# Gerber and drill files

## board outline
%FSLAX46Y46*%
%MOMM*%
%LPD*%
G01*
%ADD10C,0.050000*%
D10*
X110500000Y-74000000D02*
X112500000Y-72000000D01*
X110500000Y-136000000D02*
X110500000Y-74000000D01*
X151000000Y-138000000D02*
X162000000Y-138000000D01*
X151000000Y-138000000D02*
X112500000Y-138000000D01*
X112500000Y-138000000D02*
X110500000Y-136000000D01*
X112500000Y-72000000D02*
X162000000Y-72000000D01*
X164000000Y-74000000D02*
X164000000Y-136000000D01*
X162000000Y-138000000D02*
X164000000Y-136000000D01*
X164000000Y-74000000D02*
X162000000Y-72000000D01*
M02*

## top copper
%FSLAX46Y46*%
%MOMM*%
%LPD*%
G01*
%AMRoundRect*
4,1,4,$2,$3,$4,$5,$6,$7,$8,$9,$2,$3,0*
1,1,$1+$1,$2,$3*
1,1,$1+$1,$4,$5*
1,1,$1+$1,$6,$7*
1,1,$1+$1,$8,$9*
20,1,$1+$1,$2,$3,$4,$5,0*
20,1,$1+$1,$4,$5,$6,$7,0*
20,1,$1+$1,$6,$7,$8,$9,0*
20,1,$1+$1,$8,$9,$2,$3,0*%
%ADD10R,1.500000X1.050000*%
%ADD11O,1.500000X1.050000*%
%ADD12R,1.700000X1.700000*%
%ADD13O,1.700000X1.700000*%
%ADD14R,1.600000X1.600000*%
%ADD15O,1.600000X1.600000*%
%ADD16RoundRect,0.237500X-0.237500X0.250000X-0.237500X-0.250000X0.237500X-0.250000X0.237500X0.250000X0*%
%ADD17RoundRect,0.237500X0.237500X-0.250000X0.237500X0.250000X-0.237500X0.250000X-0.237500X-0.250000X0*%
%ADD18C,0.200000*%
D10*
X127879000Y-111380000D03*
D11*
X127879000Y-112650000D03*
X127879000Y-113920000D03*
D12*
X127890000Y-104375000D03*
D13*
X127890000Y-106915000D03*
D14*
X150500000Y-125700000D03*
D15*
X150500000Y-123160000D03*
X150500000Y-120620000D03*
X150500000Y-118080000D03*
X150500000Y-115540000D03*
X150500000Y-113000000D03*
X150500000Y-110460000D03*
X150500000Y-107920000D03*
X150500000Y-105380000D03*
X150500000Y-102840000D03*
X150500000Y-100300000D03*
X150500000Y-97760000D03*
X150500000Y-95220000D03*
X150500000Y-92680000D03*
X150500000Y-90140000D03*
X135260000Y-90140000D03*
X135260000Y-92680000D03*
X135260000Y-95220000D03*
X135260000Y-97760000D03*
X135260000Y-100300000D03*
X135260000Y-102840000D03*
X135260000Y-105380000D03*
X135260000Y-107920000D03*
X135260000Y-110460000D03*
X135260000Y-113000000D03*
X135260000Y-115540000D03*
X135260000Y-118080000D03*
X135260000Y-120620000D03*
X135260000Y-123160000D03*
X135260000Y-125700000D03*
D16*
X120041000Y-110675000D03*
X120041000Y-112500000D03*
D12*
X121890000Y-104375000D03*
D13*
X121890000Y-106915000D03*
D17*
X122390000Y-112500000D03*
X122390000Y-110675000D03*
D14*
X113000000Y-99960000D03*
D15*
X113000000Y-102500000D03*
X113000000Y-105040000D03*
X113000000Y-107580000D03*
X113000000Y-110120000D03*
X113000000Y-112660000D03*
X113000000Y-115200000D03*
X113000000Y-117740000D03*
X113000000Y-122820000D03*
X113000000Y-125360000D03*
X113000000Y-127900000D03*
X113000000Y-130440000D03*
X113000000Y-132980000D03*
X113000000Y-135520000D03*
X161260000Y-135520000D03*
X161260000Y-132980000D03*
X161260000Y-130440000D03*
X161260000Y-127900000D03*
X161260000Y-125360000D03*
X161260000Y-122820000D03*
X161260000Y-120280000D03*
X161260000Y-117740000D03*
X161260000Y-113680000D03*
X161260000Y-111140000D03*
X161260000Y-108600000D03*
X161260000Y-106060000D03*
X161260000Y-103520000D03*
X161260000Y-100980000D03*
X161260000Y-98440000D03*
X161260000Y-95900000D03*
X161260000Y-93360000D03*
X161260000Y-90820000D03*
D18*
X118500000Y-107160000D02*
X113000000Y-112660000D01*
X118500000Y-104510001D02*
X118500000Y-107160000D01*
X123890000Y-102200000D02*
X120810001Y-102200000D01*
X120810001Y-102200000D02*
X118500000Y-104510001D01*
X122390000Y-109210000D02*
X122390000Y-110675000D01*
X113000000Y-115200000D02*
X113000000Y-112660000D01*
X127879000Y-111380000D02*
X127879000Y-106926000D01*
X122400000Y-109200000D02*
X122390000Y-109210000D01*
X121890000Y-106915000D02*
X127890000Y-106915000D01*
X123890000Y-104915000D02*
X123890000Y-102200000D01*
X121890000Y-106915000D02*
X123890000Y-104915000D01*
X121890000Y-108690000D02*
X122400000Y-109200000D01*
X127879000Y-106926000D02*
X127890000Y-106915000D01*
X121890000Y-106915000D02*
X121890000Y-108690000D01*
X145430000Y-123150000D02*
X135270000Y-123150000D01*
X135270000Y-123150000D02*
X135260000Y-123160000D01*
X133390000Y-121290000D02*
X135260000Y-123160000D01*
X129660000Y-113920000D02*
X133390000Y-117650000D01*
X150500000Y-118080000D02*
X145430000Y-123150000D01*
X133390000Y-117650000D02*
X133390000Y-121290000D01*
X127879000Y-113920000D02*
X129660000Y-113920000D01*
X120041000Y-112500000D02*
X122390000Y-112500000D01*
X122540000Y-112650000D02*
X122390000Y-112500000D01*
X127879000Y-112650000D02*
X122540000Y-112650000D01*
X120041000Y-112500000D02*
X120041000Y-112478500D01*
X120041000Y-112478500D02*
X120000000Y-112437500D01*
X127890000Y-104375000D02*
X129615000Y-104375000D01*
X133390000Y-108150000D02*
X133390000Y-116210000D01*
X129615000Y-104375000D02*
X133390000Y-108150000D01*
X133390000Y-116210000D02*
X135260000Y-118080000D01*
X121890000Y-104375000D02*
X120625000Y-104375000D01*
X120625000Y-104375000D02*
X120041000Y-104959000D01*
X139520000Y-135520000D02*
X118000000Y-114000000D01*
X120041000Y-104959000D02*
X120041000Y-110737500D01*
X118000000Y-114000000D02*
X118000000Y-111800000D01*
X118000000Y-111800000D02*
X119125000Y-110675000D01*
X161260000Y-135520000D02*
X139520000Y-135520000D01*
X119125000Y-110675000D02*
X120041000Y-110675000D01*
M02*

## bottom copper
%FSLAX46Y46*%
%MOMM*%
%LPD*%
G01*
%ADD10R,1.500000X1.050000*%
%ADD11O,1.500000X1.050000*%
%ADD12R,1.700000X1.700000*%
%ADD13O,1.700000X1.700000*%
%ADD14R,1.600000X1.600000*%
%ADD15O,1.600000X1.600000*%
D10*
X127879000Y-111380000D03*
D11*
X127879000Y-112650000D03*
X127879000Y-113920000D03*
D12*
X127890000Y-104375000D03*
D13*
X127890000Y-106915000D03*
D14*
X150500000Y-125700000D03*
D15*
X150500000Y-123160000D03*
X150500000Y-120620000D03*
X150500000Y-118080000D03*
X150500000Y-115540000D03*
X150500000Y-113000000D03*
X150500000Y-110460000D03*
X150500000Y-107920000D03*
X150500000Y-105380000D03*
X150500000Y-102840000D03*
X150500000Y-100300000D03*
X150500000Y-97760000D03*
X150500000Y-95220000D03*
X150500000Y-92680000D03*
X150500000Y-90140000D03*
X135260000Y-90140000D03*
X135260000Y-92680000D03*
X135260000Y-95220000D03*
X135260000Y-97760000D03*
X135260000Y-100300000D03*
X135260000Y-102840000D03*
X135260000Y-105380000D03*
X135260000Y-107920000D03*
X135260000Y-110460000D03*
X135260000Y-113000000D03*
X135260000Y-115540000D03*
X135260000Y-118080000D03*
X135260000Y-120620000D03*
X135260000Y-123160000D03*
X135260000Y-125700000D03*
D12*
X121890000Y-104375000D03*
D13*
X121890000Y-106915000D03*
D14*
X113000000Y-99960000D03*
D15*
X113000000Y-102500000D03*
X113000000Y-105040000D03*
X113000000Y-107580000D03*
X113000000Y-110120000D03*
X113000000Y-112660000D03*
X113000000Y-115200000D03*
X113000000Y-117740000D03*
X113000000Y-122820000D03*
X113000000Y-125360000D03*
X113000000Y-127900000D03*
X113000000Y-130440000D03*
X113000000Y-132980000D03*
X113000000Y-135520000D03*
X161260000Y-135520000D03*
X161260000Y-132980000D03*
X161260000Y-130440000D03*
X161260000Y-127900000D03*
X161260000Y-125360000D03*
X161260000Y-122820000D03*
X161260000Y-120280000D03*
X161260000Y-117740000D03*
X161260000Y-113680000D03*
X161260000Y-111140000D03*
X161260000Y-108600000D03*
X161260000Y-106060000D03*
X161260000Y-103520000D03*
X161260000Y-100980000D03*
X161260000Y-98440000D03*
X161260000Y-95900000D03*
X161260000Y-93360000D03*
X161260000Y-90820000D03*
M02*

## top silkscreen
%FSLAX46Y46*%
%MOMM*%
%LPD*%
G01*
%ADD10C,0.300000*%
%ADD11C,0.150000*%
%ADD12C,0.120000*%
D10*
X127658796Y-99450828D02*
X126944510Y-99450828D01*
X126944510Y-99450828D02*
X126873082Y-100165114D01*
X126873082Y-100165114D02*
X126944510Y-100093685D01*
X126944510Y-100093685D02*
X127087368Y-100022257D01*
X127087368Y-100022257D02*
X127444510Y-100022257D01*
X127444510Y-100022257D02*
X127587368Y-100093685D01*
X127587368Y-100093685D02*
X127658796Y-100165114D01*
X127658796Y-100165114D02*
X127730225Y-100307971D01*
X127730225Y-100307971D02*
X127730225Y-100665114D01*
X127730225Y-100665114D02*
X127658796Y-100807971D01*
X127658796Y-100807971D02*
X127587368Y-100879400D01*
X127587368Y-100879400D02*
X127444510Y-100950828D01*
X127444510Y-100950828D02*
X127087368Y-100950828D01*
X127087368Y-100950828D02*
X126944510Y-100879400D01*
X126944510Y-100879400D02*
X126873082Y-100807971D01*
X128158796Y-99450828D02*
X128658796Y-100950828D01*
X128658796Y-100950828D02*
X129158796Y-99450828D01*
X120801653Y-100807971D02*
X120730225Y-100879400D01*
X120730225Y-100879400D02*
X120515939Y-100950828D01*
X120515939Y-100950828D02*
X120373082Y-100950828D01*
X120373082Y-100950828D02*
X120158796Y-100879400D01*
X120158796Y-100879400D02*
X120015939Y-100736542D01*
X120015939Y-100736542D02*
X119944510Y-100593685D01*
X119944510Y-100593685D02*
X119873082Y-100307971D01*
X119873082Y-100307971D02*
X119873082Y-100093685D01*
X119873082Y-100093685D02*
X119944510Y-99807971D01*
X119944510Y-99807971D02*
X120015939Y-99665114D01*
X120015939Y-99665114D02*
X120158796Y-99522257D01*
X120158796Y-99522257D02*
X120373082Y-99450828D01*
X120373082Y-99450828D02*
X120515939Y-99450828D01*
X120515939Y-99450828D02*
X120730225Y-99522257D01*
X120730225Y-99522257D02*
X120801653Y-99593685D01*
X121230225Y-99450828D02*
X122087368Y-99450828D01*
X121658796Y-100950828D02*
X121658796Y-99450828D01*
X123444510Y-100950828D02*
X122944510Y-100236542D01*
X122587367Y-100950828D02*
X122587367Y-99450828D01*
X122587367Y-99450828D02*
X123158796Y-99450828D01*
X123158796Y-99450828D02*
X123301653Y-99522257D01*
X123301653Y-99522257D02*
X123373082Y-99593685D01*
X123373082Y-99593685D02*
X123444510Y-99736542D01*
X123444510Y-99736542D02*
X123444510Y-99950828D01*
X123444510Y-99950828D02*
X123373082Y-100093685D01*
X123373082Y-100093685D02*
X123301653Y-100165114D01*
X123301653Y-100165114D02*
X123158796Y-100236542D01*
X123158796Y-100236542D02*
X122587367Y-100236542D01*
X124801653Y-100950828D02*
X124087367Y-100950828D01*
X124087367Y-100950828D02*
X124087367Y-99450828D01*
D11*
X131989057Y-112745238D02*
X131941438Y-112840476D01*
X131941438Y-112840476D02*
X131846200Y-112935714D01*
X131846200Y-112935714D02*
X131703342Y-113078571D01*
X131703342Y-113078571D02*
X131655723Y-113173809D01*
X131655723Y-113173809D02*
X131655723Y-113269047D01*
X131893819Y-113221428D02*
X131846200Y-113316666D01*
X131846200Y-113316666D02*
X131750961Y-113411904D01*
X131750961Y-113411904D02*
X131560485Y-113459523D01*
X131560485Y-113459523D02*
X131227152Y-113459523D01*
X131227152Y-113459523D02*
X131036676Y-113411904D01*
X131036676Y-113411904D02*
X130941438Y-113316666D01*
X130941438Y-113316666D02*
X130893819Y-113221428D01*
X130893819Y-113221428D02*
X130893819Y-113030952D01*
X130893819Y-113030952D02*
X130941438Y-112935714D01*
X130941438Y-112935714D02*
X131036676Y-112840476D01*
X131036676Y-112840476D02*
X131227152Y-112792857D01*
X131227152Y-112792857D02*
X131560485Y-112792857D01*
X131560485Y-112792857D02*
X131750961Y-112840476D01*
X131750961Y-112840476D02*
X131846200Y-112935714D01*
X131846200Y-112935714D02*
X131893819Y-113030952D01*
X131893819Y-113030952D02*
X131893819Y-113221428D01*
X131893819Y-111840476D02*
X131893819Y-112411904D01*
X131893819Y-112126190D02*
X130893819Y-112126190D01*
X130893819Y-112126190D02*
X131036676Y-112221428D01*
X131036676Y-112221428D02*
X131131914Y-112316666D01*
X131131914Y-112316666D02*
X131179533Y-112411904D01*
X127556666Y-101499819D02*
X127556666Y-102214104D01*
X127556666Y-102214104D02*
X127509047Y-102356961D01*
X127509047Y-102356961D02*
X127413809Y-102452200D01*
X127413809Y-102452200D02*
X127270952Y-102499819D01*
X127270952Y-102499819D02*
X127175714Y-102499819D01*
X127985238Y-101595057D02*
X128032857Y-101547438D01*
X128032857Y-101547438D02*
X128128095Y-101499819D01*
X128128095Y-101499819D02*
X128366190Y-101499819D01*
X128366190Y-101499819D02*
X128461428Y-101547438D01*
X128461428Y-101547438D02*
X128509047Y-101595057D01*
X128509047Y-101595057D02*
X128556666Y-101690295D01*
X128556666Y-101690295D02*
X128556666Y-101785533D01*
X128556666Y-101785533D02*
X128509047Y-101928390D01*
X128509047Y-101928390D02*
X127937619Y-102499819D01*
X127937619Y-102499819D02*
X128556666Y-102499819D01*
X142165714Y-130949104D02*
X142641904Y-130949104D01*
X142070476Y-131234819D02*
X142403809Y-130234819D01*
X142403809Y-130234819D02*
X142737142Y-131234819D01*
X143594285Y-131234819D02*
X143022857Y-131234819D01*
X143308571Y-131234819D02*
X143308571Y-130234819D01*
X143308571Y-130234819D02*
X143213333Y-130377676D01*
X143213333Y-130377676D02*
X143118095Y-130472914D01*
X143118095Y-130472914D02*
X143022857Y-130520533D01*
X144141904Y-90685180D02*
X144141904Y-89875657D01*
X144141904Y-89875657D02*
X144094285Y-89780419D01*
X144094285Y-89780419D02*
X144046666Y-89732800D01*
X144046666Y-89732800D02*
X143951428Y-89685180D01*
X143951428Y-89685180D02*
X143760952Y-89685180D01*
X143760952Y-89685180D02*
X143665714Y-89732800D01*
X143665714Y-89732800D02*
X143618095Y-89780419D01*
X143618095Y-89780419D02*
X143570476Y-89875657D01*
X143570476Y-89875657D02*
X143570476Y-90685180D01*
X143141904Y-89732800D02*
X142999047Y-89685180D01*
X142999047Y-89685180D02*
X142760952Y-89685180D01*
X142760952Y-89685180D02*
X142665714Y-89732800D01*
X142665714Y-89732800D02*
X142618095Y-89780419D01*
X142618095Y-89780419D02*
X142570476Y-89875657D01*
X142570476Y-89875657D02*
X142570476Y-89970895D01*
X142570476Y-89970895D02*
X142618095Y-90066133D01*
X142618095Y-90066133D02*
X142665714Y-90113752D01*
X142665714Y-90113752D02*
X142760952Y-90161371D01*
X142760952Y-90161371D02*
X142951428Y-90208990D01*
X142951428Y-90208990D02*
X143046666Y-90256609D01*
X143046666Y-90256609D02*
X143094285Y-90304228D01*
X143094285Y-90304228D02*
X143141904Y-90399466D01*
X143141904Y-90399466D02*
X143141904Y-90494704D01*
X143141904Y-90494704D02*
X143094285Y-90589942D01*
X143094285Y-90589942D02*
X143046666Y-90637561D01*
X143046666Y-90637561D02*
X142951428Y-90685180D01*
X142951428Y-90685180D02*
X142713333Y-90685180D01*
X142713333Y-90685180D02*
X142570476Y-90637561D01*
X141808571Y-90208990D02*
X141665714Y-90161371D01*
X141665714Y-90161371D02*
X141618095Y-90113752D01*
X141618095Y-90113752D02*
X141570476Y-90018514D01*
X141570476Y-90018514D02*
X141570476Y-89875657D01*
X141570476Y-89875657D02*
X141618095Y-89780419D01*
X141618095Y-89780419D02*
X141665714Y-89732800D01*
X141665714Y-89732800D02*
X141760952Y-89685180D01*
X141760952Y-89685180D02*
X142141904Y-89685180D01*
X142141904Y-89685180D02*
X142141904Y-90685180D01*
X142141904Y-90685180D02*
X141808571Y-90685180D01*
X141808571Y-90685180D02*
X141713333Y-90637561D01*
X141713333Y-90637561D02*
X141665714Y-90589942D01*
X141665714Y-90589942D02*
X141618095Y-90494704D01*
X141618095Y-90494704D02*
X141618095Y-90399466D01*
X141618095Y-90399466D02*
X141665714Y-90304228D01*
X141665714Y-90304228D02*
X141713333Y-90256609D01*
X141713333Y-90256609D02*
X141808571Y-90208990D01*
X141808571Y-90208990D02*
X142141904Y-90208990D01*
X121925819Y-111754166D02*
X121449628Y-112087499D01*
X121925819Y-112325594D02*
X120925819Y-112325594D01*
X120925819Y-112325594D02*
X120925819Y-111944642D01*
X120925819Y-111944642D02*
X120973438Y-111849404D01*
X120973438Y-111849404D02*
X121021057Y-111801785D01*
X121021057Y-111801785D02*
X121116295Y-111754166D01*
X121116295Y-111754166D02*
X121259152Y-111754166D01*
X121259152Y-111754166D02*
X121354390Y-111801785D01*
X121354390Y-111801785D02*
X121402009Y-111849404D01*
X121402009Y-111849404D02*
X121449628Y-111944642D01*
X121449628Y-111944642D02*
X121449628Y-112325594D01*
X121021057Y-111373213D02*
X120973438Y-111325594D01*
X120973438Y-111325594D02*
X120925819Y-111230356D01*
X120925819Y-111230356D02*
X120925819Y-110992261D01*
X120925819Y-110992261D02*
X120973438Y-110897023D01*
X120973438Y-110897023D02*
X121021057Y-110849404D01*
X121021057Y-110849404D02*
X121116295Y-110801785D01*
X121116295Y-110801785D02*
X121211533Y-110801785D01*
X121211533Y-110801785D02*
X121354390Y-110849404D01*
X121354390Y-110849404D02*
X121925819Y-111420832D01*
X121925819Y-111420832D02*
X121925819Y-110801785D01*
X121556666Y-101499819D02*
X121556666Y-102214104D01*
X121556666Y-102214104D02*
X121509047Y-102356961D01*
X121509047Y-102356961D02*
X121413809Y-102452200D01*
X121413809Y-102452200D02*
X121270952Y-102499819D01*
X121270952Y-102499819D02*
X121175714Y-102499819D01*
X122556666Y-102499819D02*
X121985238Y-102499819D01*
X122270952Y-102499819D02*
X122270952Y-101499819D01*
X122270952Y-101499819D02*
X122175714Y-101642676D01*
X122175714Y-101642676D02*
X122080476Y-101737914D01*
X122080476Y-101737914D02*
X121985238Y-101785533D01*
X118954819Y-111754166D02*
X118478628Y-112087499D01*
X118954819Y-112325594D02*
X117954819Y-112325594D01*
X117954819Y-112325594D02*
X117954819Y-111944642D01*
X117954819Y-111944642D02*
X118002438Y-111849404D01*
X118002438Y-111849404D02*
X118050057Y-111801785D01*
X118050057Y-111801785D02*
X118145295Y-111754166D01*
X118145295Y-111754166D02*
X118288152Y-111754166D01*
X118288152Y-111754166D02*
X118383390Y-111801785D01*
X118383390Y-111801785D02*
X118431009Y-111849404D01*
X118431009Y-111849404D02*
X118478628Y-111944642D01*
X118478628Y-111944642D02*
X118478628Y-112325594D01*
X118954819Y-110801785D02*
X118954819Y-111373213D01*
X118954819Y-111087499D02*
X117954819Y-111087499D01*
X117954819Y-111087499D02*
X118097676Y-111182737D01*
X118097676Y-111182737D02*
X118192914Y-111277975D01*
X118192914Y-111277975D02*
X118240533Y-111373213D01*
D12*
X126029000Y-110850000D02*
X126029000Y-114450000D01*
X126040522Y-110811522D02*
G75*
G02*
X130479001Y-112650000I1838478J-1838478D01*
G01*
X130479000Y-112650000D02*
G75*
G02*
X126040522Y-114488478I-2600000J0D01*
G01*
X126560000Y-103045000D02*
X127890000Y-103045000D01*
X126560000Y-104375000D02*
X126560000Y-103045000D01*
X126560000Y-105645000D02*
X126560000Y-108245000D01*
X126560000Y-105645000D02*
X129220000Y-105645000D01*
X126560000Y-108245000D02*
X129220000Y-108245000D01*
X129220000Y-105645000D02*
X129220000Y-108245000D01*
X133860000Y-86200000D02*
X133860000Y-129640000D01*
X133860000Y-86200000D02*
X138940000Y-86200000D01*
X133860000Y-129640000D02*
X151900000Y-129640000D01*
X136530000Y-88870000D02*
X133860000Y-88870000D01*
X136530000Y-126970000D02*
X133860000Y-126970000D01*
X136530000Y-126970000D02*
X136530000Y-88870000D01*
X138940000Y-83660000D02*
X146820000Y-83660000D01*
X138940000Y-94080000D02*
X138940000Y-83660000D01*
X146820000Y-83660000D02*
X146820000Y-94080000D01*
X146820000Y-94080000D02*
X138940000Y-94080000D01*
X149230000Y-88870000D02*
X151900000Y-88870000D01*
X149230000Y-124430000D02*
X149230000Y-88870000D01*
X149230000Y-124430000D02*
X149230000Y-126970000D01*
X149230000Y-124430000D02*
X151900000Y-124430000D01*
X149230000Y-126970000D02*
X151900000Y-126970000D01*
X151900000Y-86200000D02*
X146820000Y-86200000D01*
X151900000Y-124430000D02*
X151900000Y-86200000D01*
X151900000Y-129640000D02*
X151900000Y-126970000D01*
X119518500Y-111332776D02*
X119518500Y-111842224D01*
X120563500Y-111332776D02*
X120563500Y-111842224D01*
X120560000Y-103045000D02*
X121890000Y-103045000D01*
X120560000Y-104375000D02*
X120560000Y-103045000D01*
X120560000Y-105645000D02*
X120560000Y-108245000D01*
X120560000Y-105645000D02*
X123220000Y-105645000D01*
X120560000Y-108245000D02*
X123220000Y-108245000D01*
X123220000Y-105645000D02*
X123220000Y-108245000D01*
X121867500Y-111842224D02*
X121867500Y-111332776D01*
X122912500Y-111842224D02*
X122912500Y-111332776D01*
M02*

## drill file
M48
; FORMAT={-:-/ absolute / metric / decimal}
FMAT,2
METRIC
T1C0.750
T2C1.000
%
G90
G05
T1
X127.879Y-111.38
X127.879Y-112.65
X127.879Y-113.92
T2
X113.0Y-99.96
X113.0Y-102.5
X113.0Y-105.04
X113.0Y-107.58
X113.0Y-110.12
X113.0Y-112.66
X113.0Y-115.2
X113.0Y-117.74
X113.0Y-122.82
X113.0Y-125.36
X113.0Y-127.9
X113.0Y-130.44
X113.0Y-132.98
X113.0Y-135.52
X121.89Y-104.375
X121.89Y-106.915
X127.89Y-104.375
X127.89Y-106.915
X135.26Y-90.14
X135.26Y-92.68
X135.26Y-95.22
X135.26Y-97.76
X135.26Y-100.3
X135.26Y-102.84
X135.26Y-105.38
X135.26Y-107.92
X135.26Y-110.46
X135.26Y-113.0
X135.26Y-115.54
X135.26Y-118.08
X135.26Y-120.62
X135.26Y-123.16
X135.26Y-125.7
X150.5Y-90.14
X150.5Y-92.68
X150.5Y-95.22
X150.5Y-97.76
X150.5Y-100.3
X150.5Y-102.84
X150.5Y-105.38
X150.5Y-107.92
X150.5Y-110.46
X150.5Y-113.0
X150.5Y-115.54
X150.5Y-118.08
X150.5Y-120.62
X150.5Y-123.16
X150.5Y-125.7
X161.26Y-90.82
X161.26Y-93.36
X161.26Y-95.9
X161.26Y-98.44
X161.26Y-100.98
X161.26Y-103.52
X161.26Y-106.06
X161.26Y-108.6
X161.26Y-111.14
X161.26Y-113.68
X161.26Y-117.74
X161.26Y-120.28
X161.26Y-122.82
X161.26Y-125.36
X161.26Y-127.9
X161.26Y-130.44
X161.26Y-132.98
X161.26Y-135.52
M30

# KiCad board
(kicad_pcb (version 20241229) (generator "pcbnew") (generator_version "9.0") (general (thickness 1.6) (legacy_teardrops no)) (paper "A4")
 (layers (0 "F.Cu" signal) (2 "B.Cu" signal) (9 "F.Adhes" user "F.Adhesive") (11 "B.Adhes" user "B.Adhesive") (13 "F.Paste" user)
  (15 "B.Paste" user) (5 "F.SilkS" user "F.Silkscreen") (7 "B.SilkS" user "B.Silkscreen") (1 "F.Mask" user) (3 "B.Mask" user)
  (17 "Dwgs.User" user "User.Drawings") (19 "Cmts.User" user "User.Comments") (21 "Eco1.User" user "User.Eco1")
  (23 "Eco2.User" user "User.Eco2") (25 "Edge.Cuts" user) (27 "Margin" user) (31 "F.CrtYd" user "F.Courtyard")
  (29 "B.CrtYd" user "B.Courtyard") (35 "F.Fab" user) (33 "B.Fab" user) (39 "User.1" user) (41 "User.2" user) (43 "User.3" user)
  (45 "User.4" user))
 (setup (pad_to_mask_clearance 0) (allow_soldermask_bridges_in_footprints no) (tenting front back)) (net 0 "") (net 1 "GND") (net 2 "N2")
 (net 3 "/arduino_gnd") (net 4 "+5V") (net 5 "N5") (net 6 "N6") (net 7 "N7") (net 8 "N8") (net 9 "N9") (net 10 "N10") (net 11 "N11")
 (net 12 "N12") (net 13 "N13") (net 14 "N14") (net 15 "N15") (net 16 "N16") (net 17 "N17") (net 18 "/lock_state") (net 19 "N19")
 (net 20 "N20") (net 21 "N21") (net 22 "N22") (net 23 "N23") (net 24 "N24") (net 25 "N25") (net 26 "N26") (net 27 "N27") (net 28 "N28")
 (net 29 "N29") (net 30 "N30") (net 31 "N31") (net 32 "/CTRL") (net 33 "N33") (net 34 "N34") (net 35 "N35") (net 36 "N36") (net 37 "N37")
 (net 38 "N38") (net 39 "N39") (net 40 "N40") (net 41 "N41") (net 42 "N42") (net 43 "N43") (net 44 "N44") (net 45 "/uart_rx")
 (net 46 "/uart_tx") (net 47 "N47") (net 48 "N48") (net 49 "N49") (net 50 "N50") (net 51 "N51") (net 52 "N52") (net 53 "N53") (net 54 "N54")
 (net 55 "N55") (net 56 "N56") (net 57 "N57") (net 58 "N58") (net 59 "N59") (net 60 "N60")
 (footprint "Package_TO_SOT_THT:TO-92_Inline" (layer "F.Cu") (at 127.879 111.38 -90)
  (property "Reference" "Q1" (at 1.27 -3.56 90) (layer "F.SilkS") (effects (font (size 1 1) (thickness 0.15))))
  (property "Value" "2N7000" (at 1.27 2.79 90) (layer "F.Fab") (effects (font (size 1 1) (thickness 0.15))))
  (fp_line (start -0.53 1.85) (end 3.07 1.85) (stroke (width 0.12) (type solid)) (layer "F.SilkS"))
  (fp_arc (start -0.568478 1.838478) (mid -1.132087 -0.994977) (end 1.27 -2.6) (stroke (width 0.12) (type solid)) (layer "F.SilkS"))
  (fp_arc (start 1.27 -2.6) (mid 3.672087 -0.994977) (end 3.108478 1.838478) (stroke (width 0.12) (type solid)) (layer "F.SilkS"))
  (pad "1" thru_hole rect (at 0 0 270) (size 1.05 1.5) (drill 0.75) (layers "*.Cu" "*.Mask") (remove_unused_layers no) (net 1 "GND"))
  (pad "2" thru_hole oval (at 1.27 0 270) (size 1.05 1.5) (drill 0.75) (layers "*.Cu" "*.Mask") (remove_unused_layers no) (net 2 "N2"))
  (pad "3" thru_hole oval (at 2.54 0 270) (size 1.05 1.5) (drill 0.75) (layers "*.Cu" "*.Mask") (remove_unused_layers no)
   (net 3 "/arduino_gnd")))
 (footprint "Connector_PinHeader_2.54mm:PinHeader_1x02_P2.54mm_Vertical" (layer "F.Cu") (at 127.89 104.375)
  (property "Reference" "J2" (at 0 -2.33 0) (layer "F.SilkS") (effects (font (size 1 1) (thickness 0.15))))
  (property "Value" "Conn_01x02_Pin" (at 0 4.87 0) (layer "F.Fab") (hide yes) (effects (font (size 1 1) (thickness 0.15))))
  (fp_line (start -1.33 -1.33) (end 0 -1.33) (stroke (width 0.12) (type solid)) (layer "F.SilkS"))
  (fp_line (start -1.33 0) (end -1.33 -1.33) (stroke (width 0.12) (type solid)) (layer "F.SilkS"))
  (fp_line (start -1.33 1.27) (end -1.33 3.87) (stroke (width 0.12) (type solid)) (layer "F.SilkS"))
  (fp_line (start -1.33 1.27) (end 1.33 1.27) (stroke (width 0.12) (type solid)) (layer "F.SilkS"))
  (fp_line (start -1.33 3.87) (end 1.33 3.87) (stroke (width 0.12) (type solid)) (layer "F.SilkS"))
  (fp_line (start 1.33 1.27) (end 1.33 3.87) (stroke (width 0.12) (type solid)) (layer "F.SilkS"))
  (pad "1" thru_hole rect (at 0 0) (size 1.7 1.7) (drill 1) (layers "*.Cu" "*.Mask") (remove_unused_layers no) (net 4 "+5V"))
  (pad "2" thru_hole oval (at 0 2.54) (size 1.7 1.7) (drill 1) (layers "*.Cu" "*.Mask") (remove_unused_layers no) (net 1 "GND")))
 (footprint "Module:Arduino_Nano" (layer "F.Cu") (at 150.5 125.7 180)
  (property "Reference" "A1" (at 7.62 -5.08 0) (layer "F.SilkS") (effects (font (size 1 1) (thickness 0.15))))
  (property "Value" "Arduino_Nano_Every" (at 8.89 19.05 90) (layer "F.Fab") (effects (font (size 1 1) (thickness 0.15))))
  (fp_line (start 16.64 39.5) (end 16.64 -3.94) (stroke (width 0.12) (type solid)) (layer "F.SilkS"))
  (fp_line (start 16.64 39.5) (end 11.56 39.5) (stroke (width 0.12) (type solid)) (layer "F.SilkS"))
  (fp_line (start 16.64 -3.94) (end -1.4 -3.94) (stroke (width 0.12) (type solid)) (layer "F.SilkS"))
  (fp_line (start 13.97 36.83) (end 16.64 36.83) (stroke (width 0.12) (type solid)) (layer "F.SilkS"))
  (fp_line (start 13.97 -1.27) (end 16.64 -1.27) (stroke (width 0.12) (type solid)) (layer "F.SilkS"))
  (fp_line (start 13.97 -1.27) (end 13.97 36.83) (stroke (width 0.12) (type solid)) (layer "F.SilkS"))
  (fp_line (start 11.56 42.04) (end 3.68 42.04) (stroke (width 0.12) (type solid)) (layer "F.SilkS"))
  (fp_line (start 11.56 31.62) (end 11.56 42.04) (stroke (width 0.12) (type solid)) (layer "F.SilkS"))
  (fp_line (start 3.68 42.04) (end 3.68 31.62) (stroke (width 0.12) (type solid)) (layer "F.SilkS"))
  (fp_line (start 3.68 31.62) (end 11.56 31.62) (stroke (width 0.12) (type solid)) (layer "F.SilkS"))
  (fp_line (start 1.27 36.83) (end -1.4 36.83) (stroke (width 0.12) (type solid)) (layer "F.SilkS"))
  (fp_line (start 1.27 1.27) (end 1.27 36.83) (stroke (width 0.12) (type solid)) (layer "F.SilkS"))
  (fp_line (start 1.27 1.27) (end 1.27 -1.27) (stroke (width 0.12) (type solid)) (layer "F.SilkS"))
  (fp_line (start 1.27 1.27) (end -1.4 1.27) (stroke (width 0.12) (type solid)) (layer "F.SilkS"))
  (fp_line (start 1.27 -1.27) (end -1.4 -1.27) (stroke (width 0.12) (type solid)) (layer "F.SilkS"))
  (fp_line (start -1.4 39.5) (end 3.68 39.5) (stroke (width 0.12) (type solid)) (layer "F.SilkS"))
  (fp_line (start -1.4 1.27) (end -1.4 39.5) (stroke (width 0.12) (type solid)) (layer "F.SilkS"))
  (fp_line (start -1.4 -3.94) (end -1.4 -1.27) (stroke (width 0.12) (type solid)) (layer "F.SilkS"))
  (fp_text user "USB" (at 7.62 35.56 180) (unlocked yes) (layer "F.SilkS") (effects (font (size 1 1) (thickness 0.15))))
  (pad "1" thru_hole rect (at 0 0 180) (size 1.6 1.6) (drill 1) (layers "*.Cu" "*.Mask") (remove_unused_layers no) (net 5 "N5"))
  (pad "2" thru_hole oval (at 0 2.54 180) (size 1.6 1.6) (drill 1) (layers "*.Cu" "*.Mask") (remove_unused_layers no) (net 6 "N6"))
  (pad "3" thru_hole oval (at 0 5.08 180) (size 1.6 1.6) (drill 1) (layers "*.Cu" "*.Mask") (remove_unused_layers no) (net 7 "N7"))
  (pad "4" thru_hole oval (at 0 7.62 180) (size 1.6 1.6) (drill 1) (layers "*.Cu" "*.Mask") (remove_unused_layers no) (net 3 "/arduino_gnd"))
  (pad "5" thru_hole oval (at 0 10.16 180) (size 1.6 1.6) (drill 1) (layers "*.Cu" "*.Mask") (remove_unused_layers no) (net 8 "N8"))
  (pad "6" thru_hole oval (at 0 12.7 180) (size 1.6 1.6) (drill 1) (layers "*.Cu" "*.Mask") (remove_unused_layers no) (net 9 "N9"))
  (pad "7" thru_hole oval (at 0 15.24 180) (size 1.6 1.6) (drill 1) (layers "*.Cu" "*.Mask") (remove_unused_layers no) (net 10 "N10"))
  (pad "8" thru_hole oval (at 0 17.78 180) (size 1.6 1.6) (drill 1) (layers "*.Cu" "*.Mask") (remove_unused_layers no) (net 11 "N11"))
  (pad "9" thru_hole oval (at 0 20.32 180) (size 1.6 1.6) (drill 1) (layers "*.Cu" "*.Mask") (remove_unused_layers no) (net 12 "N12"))
  (pad "10" thru_hole oval (at 0 22.86 180) (size 1.6 1.6) (drill 1) (layers "*.Cu" "*.Mask") (remove_unused_layers no) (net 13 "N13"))
  (pad "11" thru_hole oval (at 0 25.4 180) (size 1.6 1.6) (drill 1) (layers "*.Cu" "*.Mask") (remove_unused_layers no) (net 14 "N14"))
  (pad "12" thru_hole oval (at 0 27.94 180) (size 1.6 1.6) (drill 1) (layers "*.Cu" "*.Mask") (remove_unused_layers no) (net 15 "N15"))
  (pad "13" thru_hole oval (at 0 30.48 180) (size 1.6 1.6) (drill 1) (layers "*.Cu" "*.Mask") (remove_unused_layers no) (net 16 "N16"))
  (pad "14" thru_hole oval (at 0 33.02 180) (size 1.6 1.6) (drill 1) (layers "*.Cu" "*.Mask") (remove_unused_layers no) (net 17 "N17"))
  (pad "15" thru_hole oval (at 0 35.56 180) (size 1.6 1.6) (drill 1) (layers "*.Cu" "*.Mask") (remove_unused_layers no)
   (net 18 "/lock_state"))
  (pad "16" thru_hole oval (at 15.24 35.56 180) (size 1.6 1.6) (drill 1) (layers "*.Cu" "*.Mask") (remove_unused_layers no) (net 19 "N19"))
  (pad "17" thru_hole oval (at 15.24 33.02 180) (size 1.6 1.6) (drill 1) (layers "*.Cu" "*.Mask") (remove_unused_layers no) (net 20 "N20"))
  (pad "18" thru_hole oval (at 15.24 30.48 180) (size 1.6 1.6) (drill 1) (layers "*.Cu" "*.Mask") (remove_unused_layers no) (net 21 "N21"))
  (pad "19" thru_hole oval (at 15.24 27.94 180) (size 1.6 1.6) (drill 1) (layers "*.Cu" "*.Mask") (remove_unused_layers no) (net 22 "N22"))
  (pad "20" thru_hole oval (at 15.24 25.4 180) (size 1.6 1.6) (drill 1) (layers "*.Cu" "*.Mask") (remove_unused_layers no) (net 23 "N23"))
  (pad "21" thru_hole oval (at 15.24 22.86 180) (size 1.6 1.6) (drill 1) (layers "*.Cu" "*.Mask") (remove_unused_layers no) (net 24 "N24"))
  (pad "22" thru_hole oval (at 15.24 20.32 180) (size 1.6 1.6) (drill 1) (layers "*.Cu" "*.Mask") (remove_unused_layers no) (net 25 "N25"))
  (pad "23" thru_hole oval (at 15.24 17.78 180) (size 1.6 1.6) (drill 1) (layers "*.Cu" "*.Mask") (remove_unused_layers no) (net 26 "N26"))
  (pad "24" thru_hole oval (at 15.24 15.24 180) (size 1.6 1.6) (drill 1) (layers "*.Cu" "*.Mask") (remove_unused_layers no) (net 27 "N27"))
  (pad "25" thru_hole oval (at 15.24 12.7 180) (size 1.6 1.6) (drill 1) (layers "*.Cu" "*.Mask") (remove_unused_layers no) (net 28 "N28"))
  (pad "26" thru_hole oval (at 15.24 10.16 180) (size 1.6 1.6) (drill 1) (layers "*.Cu" "*.Mask") (remove_unused_layers no) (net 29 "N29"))
  (pad "27" thru_hole oval (at 15.24 7.62 180) (size 1.6 1.6) (drill 1) (layers "*.Cu" "*.Mask") (remove_unused_layers no) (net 4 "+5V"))
  (pad "28" thru_hole oval (at 15.24 5.08 180) (size 1.6 1.6) (drill 1) (layers "*.Cu" "*.Mask") (remove_unused_layers no) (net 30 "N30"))
  (pad "29" thru_hole oval (at 15.24 2.54 180) (size 1.6 1.6) (drill 1) (layers "*.Cu" "*.Mask") (remove_unused_layers no)
   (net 3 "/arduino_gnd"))
  (pad "30" thru_hole oval (at 15.24 0 180) (size 1.6 1.6) (drill 1) (layers "*.Cu" "*.Mask") (remove_unused_layers no) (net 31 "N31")))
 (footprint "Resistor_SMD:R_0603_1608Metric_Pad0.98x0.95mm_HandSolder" (layer "F.Cu") (at 120.041 111.5875 -90)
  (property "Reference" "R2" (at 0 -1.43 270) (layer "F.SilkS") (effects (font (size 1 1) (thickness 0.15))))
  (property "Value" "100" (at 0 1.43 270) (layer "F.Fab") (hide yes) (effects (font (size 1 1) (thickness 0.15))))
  (fp_line (start -0.254724 0.5225) (end 0.254724 0.5225) (stroke (width 0.12) (type solid)) (layer "F.SilkS"))
  (fp_line (start -0.254724 -0.5225) (end 0.254724 -0.5225) (stroke (width 0.12) (type solid)) (layer "F.SilkS"))
  (pad "1" smd roundrect (at -0.9125 0 270) (size 0.975 0.95) (layers "F.Cu" "F.Mask" "F.Paste") (roundrect_rratio 0.25) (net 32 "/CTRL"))
  (pad "2" smd roundrect (at 0.9125 0 270) (size 0.975 0.95) (layers "F.Cu" "F.Mask" "F.Paste") (roundrect_rratio 0.25) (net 2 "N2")))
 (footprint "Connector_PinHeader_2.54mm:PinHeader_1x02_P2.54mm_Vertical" (layer "F.Cu") (at 121.89 104.375)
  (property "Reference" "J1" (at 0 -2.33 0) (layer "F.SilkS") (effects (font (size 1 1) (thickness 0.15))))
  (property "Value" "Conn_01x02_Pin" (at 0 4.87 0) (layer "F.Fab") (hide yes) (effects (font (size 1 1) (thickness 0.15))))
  (fp_line (start -1.33 -1.33) (end 0 -1.33) (stroke (width 0.12) (type solid)) (layer "F.SilkS"))
  (fp_line (start -1.33 0) (end -1.33 -1.33) (stroke (width 0.12) (type solid)) (layer "F.SilkS"))
  (fp_line (start -1.33 1.27) (end -1.33 3.87) (stroke (width 0.12) (type solid)) (layer "F.SilkS"))
  (fp_line (start -1.33 1.27) (end 1.33 1.27) (stroke (width 0.12) (type solid)) (layer "F.SilkS"))
  (fp_line (start -1.33 3.87) (end 1.33 3.87) (stroke (width 0.12) (type solid)) (layer "F.SilkS"))
  (fp_line (start 1.33 1.27) (end 1.33 3.87) (stroke (width 0.12) (type solid)) (layer "F.SilkS"))
  (pad "1" thru_hole rect (at 0 0) (size 1.7 1.7) (drill 1) (layers "*.Cu" "*.Mask") (remove_unused_layers no) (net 32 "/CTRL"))
  (pad "2" thru_hole oval (at 0 2.54) (size 1.7 1.7) (drill 1) (layers "*.Cu" "*.Mask") (remove_unused_layers no) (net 1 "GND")))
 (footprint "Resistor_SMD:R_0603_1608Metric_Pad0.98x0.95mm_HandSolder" (layer "F.Cu") (at 122.39 111.5875 90)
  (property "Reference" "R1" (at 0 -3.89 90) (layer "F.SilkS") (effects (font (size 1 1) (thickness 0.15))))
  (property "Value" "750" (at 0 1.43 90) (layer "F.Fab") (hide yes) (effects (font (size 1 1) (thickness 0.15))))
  (fp_line (start -0.254724 -0.5225) (end 0.254724 -0.5225) (stroke (width 0.12) (type solid)) (layer "F.SilkS"))
  (fp_line (start -0.254724 0.5225) (end 0.254724 0.5225) (stroke (width 0.12) (type solid)) (layer "F.SilkS"))
  (pad "1" smd roundrect (at -0.9125 0 90) (size 0.975 0.95) (layers "F.Cu" "F.Mask" "F.Paste") (roundrect_rratio 0.25) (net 2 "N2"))
  (pad "2" smd roundrect (at 0.9125 0 90) (size 0.975 0.95) (layers "F.Cu" "F.Mask" "F.Paste") (roundrect_rratio 0.25) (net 1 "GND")))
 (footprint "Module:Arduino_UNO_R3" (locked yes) (layer "B.Cu") (at 113 99.96 -90)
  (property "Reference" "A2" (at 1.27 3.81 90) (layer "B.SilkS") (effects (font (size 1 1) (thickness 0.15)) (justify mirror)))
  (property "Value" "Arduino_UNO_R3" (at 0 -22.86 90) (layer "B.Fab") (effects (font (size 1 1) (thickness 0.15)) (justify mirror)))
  (pad "1" thru_hole rect (at 0 0 180) (size 1.6 1.6) (drill 1) (layers "*.Cu" "*.Mask") (remove_unused_layers no) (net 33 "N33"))
  (pad "2" thru_hole oval (at 2.54 0 180) (size 1.6 1.6) (drill 1) (layers "*.Cu" "*.Mask") (remove_unused_layers no) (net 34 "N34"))
  (pad "3" thru_hole oval (at 5.08 0 180) (size 1.6 1.6) (drill 1) (layers "*.Cu" "*.Mask") (remove_unused_layers no) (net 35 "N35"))
  (pad "4" thru_hole oval (at 7.62 0 180) (size 1.6 1.6) (drill 1) (layers "*.Cu" "*.Mask") (remove_unused_layers no) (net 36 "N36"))
  (pad "5" thru_hole oval (at 10.16 0 180) (size 1.6 1.6) (drill 1) (layers "*.Cu" "*.Mask") (remove_unused_layers no) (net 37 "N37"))
  (pad "6" thru_hole oval (at 12.7 0 180) (size 1.6 1.6) (drill 1) (layers "*.Cu" "*.Mask") (remove_unused_layers no) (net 1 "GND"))
  (pad "7" thru_hole oval (at 15.24 0 180) (size 1.6 1.6) (drill 1) (layers "*.Cu" "*.Mask") (remove_unused_layers no) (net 1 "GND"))
  (pad "8" thru_hole oval (at 17.78 0 180) (size 1.6 1.6) (drill 1) (layers "*.Cu" "*.Mask") (remove_unused_layers no) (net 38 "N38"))
  (pad "9" thru_hole oval (at 22.86 0 180) (size 1.6 1.6) (drill 1) (layers "*.Cu" "*.Mask") (remove_unused_layers no) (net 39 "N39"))
  (pad "10" thru_hole oval (at 25.4 0 180) (size 1.6 1.6) (drill 1) (layers "*.Cu" "*.Mask") (remove_unused_layers no) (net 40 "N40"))
  (pad "11" thru_hole oval (at 27.94 0 180) (size 1.6 1.6) (drill 1) (layers "*.Cu" "*.Mask") (remove_unused_layers no) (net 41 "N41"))
  (pad "12" thru_hole oval (at 30.48 0 180) (size 1.6 1.6) (drill 1) (layers "*.Cu" "*.Mask") (remove_unused_layers no) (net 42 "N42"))
  (pad "13" thru_hole oval (at 33.02 0 180) (size 1.6 1.6) (drill 1) (layers "*.Cu" "*.Mask") (remove_unused_layers no) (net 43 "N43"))
  (pad "14" thru_hole oval (at 35.56 0 180) (size 1.6 1.6) (drill 1) (layers "*.Cu" "*.Mask") (remove_unused_layers no) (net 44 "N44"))
  (pad "15" thru_hole oval (at 35.56 -48.26 180) (size 1.6 1.6) (drill 1) (layers "*.Cu" "*.Mask") (remove_unused_layers no)
   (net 32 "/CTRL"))
  (pad "16" thru_hole oval (at 33.02 -48.26 180) (size 1.6 1.6) (drill 1) (layers "*.Cu" "*.Mask") (remove_unused_layers no)
   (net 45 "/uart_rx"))
  (pad "17" thru_hole oval (at 30.48 -48.26 180) (size 1.6 1.6) (drill 1) (layers "*.Cu" "*.Mask") (remove_unused_layers no)
   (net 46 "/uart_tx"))
  (pad "18" thru_hole oval (at 27.94 -48.26 180) (size 1.6 1.6) (drill 1) (layers "*.Cu" "*.Mask") (remove_unused_layers no) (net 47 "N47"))
  (pad "19" thru_hole oval (at 25.4 -48.26 180) (size 1.6 1.6) (drill 1) (layers "*.Cu" "*.Mask") (remove_unused_layers no) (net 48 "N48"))
  (pad "20" thru_hole oval (at 22.86 -48.26 180) (size 1.6 1.6) (drill 1) (layers "*.Cu" "*.Mask") (remove_unused_layers no) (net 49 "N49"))
  (pad "21" thru_hole oval (at 20.32 -48.26 180) (size 1.6 1.6) (drill 1) (layers "*.Cu" "*.Mask") (remove_unused_layers no) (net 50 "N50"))
  (pad "22" thru_hole oval (at 17.78 -48.26 180) (size 1.6 1.6) (drill 1) (layers "*.Cu" "*.Mask") (remove_unused_layers no) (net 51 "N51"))
  (pad "23" thru_hole oval (at 13.72 -48.26 180) (size 1.6 1.6) (drill 1) (layers "*.Cu" "*.Mask") (remove_unused_layers no) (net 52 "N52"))
  (pad "24" thru_hole oval (at 11.18 -48.26 180) (size 1.6 1.6) (drill 1) (layers "*.Cu" "*.Mask") (remove_unused_layers no) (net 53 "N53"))
  (pad "25" thru_hole oval (at 8.64 -48.26 180) (size 1.6 1.6) (drill 1) (layers "*.Cu" "*.Mask") (remove_unused_layers no) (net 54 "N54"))
  (pad "26" thru_hole oval (at 6.1 -48.26 180) (size 1.6 1.6) (drill 1) (layers "*.Cu" "*.Mask") (remove_unused_layers no) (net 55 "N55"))
  (pad "27" thru_hole oval (at 3.56 -48.26 180) (size 1.6 1.6) (drill 1) (layers "*.Cu" "*.Mask") (remove_unused_layers no) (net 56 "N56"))
  (pad "28" thru_hole oval (at 1.02 -48.26 180) (size 1.6 1.6) (drill 1) (layers "*.Cu" "*.Mask") (remove_unused_layers no) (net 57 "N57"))
  (pad "29" thru_hole oval (at -1.52 -48.26 180) (size 1.6 1.6) (drill 1) (layers "*.Cu" "*.Mask") (remove_unused_layers no) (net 1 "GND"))
  (pad "30" thru_hole oval (at -4.06 -48.26 180) (size 1.6 1.6) (drill 1) (layers "*.Cu" "*.Mask") (remove_unused_layers no) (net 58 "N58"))
  (pad "31" thru_hole oval (at -6.6 -48.26 180) (size 1.6 1.6) (drill 1) (layers "*.Cu" "*.Mask") (remove_unused_layers no) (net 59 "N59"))
  (pad "32" thru_hole oval (at -9.14 -48.26 180) (size 1.6 1.6) (drill 1) (layers "*.Cu" "*.Mask") (remove_unused_layers no) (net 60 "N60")))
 (gr_line (start 110.5 74) (end 112.5 72) (stroke (width 0.05) (type default)) (layer "Edge.Cuts"))
 (gr_line (start 110.5 136) (end 110.5 74) (stroke (width 0.05) (type default)) (layer "Edge.Cuts"))
 (gr_line (start 151 138) (end 162 138) (stroke (width 0.05) (type default)) (layer "Edge.Cuts"))
 (gr_line (start 151 138) (end 112.5 138) (stroke (width 0.05) (type default)) (layer "Edge.Cuts"))
 (gr_line (start 112.5 138) (end 110.5 136) (stroke (width 0.05) (type default)) (layer "Edge.Cuts"))
 (gr_line (start 112.5 72) (end 162 72) (stroke (width 0.05) (type default)) (layer "Edge.Cuts"))
 (gr_line (start 164 74) (end 164 136) (stroke (width 0.05) (type default)) (layer "Edge.Cuts"))
 (gr_line (start 162 138) (end 164 136) (stroke (width 0.05) (type default)) (layer "Edge.Cuts"))
 (gr_line (start 164 74) (end 162 72) (stroke (width 0.05) (type default)) (layer "Edge.Cuts"))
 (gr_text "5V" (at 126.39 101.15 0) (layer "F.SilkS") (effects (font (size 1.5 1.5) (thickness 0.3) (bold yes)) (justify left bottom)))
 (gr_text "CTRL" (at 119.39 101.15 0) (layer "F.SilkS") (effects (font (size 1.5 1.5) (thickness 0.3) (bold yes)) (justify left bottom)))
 (segment (start 118.5 107.16) (end 113 112.66) (width 0.2) (layer "F.Cu") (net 1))
 (segment (start 118.5 104.510001) (end 118.5 107.16) (width 0.2) (layer "F.Cu") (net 1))
 (segment (start 123.89 102.2) (end 120.810001 102.2) (width 0.2) (layer "F.Cu") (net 1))
 (segment (start 120.810001 102.2) (end 118.5 104.510001) (width 0.2) (layer "F.Cu") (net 1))
 (segment (start 122.39 109.21) (end 122.39 110.675) (width 0.2) (layer "F.Cu") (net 1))
 (segment (start 113 115.2) (end 113 112.66) (width 0.2) (layer "F.Cu") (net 1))
 (segment (start 127.879 111.38) (end 127.879 106.926) (width 0.2) (layer "F.Cu") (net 1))
 (segment (start 122.4 109.2) (end 122.39 109.21) (width 0.2) (layer "F.Cu") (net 1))
 (segment (start 121.89 106.915) (end 127.89 106.915) (width 0.2) (layer "F.Cu") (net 1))
 (segment (start 123.89 104.915) (end 123.89 102.2) (width 0.2) (layer "F.Cu") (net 1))
 (segment (start 121.89 106.915) (end 123.89 104.915) (width 0.2) (layer "F.Cu") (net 1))
 (segment (start 121.89 108.69) (end 122.4 109.2) (width 0.2) (layer "F.Cu") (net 1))
 (segment (start 127.879 106.926) (end 127.89 106.915) (width 0.2) (layer "F.Cu") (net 1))
 (segment (start 121.89 106.915) (end 121.89 108.69) (width 0.2) (layer "F.Cu") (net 1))
 (segment (start 145.43 123.15) (end 135.27 123.15) (width 0.2) (layer "F.Cu") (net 3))
 (segment (start 135.27 123.15) (end 135.26 123.16) (width 0.2) (layer "F.Cu") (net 3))
 (segment (start 133.39 121.29) (end 135.26 123.16) (width 0.2) (layer "F.Cu") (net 3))
 (segment (start 129.66 113.92) (end 133.39 117.65) (width 0.2) (layer "F.Cu") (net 3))
 (segment (start 150.5 118.08) (end 145.43 123.15) (width 0.2) (layer "F.Cu") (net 3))
 (segment (start 133.39 117.65) (end 133.39 121.29) (width 0.2) (layer "F.Cu") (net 3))
 (segment (start 127.879 113.92) (end 129.66 113.92) (width 0.2) (layer "F.Cu") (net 3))
 (segment (start 120.041 112.5) (end 122.39 112.5) (width 0.2) (layer "F.Cu") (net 2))
 (segment (start 122.54 112.65) (end 122.39 112.5) (width 0.2) (layer "F.Cu") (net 2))
 (segment (start 127.879 112.65) (end 122.54 112.65) (width 0.2) (layer "F.Cu") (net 2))
 (segment (start 120.041 112.5) (end 120.041 112.4785) (width 0.2) (layer "F.Cu") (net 2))
 (segment (start 120.041 112.4785) (end 120 112.4375) (width 0.2) (layer "F.Cu") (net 2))
 (segment (start 127.89 104.375) (end 129.615 104.375) (width 0.2) (layer "F.Cu") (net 4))
 (segment (start 133.39 108.15) (end 133.39 116.21) (width 0.2) (layer "F.Cu") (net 4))
 (segment (start 129.615 104.375) (end 133.39 108.15) (width 0.2) (layer "F.Cu") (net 4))
 (segment (start 133.39 116.21) (end 135.26 118.08) (width 0.2) (layer "F.Cu") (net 4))
 (segment (start 121.89 104.375) (end 120.625 104.375) (width 0.2) (layer "F.Cu") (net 32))
 (segment (start 120.625 104.375) (end 120.041 104.959) (width 0.2) (layer "F.Cu") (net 32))
 (segment (start 139.52 135.52) (end 118 114) (width 0.2) (layer "F.Cu") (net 32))
 (segment (start 120.041 104.959) (end 120.041 110.7375) (width 0.2) (layer "F.Cu") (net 32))
 (segment (start 118 114) (end 118 111.8) (width 0.2) (layer "F.Cu") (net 32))
 (segment (start 118 111.8) (end 119.125 110.675) (width 0.2) (layer "F.Cu") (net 32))
 (segment (start 161.26 135.52) (end 139.52 135.52) (width 0.2) (layer "F.Cu") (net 32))
 (segment (start 119.125 110.675) (end 120.041 110.675) (width 0.2) (layer "F.Cu") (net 32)))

